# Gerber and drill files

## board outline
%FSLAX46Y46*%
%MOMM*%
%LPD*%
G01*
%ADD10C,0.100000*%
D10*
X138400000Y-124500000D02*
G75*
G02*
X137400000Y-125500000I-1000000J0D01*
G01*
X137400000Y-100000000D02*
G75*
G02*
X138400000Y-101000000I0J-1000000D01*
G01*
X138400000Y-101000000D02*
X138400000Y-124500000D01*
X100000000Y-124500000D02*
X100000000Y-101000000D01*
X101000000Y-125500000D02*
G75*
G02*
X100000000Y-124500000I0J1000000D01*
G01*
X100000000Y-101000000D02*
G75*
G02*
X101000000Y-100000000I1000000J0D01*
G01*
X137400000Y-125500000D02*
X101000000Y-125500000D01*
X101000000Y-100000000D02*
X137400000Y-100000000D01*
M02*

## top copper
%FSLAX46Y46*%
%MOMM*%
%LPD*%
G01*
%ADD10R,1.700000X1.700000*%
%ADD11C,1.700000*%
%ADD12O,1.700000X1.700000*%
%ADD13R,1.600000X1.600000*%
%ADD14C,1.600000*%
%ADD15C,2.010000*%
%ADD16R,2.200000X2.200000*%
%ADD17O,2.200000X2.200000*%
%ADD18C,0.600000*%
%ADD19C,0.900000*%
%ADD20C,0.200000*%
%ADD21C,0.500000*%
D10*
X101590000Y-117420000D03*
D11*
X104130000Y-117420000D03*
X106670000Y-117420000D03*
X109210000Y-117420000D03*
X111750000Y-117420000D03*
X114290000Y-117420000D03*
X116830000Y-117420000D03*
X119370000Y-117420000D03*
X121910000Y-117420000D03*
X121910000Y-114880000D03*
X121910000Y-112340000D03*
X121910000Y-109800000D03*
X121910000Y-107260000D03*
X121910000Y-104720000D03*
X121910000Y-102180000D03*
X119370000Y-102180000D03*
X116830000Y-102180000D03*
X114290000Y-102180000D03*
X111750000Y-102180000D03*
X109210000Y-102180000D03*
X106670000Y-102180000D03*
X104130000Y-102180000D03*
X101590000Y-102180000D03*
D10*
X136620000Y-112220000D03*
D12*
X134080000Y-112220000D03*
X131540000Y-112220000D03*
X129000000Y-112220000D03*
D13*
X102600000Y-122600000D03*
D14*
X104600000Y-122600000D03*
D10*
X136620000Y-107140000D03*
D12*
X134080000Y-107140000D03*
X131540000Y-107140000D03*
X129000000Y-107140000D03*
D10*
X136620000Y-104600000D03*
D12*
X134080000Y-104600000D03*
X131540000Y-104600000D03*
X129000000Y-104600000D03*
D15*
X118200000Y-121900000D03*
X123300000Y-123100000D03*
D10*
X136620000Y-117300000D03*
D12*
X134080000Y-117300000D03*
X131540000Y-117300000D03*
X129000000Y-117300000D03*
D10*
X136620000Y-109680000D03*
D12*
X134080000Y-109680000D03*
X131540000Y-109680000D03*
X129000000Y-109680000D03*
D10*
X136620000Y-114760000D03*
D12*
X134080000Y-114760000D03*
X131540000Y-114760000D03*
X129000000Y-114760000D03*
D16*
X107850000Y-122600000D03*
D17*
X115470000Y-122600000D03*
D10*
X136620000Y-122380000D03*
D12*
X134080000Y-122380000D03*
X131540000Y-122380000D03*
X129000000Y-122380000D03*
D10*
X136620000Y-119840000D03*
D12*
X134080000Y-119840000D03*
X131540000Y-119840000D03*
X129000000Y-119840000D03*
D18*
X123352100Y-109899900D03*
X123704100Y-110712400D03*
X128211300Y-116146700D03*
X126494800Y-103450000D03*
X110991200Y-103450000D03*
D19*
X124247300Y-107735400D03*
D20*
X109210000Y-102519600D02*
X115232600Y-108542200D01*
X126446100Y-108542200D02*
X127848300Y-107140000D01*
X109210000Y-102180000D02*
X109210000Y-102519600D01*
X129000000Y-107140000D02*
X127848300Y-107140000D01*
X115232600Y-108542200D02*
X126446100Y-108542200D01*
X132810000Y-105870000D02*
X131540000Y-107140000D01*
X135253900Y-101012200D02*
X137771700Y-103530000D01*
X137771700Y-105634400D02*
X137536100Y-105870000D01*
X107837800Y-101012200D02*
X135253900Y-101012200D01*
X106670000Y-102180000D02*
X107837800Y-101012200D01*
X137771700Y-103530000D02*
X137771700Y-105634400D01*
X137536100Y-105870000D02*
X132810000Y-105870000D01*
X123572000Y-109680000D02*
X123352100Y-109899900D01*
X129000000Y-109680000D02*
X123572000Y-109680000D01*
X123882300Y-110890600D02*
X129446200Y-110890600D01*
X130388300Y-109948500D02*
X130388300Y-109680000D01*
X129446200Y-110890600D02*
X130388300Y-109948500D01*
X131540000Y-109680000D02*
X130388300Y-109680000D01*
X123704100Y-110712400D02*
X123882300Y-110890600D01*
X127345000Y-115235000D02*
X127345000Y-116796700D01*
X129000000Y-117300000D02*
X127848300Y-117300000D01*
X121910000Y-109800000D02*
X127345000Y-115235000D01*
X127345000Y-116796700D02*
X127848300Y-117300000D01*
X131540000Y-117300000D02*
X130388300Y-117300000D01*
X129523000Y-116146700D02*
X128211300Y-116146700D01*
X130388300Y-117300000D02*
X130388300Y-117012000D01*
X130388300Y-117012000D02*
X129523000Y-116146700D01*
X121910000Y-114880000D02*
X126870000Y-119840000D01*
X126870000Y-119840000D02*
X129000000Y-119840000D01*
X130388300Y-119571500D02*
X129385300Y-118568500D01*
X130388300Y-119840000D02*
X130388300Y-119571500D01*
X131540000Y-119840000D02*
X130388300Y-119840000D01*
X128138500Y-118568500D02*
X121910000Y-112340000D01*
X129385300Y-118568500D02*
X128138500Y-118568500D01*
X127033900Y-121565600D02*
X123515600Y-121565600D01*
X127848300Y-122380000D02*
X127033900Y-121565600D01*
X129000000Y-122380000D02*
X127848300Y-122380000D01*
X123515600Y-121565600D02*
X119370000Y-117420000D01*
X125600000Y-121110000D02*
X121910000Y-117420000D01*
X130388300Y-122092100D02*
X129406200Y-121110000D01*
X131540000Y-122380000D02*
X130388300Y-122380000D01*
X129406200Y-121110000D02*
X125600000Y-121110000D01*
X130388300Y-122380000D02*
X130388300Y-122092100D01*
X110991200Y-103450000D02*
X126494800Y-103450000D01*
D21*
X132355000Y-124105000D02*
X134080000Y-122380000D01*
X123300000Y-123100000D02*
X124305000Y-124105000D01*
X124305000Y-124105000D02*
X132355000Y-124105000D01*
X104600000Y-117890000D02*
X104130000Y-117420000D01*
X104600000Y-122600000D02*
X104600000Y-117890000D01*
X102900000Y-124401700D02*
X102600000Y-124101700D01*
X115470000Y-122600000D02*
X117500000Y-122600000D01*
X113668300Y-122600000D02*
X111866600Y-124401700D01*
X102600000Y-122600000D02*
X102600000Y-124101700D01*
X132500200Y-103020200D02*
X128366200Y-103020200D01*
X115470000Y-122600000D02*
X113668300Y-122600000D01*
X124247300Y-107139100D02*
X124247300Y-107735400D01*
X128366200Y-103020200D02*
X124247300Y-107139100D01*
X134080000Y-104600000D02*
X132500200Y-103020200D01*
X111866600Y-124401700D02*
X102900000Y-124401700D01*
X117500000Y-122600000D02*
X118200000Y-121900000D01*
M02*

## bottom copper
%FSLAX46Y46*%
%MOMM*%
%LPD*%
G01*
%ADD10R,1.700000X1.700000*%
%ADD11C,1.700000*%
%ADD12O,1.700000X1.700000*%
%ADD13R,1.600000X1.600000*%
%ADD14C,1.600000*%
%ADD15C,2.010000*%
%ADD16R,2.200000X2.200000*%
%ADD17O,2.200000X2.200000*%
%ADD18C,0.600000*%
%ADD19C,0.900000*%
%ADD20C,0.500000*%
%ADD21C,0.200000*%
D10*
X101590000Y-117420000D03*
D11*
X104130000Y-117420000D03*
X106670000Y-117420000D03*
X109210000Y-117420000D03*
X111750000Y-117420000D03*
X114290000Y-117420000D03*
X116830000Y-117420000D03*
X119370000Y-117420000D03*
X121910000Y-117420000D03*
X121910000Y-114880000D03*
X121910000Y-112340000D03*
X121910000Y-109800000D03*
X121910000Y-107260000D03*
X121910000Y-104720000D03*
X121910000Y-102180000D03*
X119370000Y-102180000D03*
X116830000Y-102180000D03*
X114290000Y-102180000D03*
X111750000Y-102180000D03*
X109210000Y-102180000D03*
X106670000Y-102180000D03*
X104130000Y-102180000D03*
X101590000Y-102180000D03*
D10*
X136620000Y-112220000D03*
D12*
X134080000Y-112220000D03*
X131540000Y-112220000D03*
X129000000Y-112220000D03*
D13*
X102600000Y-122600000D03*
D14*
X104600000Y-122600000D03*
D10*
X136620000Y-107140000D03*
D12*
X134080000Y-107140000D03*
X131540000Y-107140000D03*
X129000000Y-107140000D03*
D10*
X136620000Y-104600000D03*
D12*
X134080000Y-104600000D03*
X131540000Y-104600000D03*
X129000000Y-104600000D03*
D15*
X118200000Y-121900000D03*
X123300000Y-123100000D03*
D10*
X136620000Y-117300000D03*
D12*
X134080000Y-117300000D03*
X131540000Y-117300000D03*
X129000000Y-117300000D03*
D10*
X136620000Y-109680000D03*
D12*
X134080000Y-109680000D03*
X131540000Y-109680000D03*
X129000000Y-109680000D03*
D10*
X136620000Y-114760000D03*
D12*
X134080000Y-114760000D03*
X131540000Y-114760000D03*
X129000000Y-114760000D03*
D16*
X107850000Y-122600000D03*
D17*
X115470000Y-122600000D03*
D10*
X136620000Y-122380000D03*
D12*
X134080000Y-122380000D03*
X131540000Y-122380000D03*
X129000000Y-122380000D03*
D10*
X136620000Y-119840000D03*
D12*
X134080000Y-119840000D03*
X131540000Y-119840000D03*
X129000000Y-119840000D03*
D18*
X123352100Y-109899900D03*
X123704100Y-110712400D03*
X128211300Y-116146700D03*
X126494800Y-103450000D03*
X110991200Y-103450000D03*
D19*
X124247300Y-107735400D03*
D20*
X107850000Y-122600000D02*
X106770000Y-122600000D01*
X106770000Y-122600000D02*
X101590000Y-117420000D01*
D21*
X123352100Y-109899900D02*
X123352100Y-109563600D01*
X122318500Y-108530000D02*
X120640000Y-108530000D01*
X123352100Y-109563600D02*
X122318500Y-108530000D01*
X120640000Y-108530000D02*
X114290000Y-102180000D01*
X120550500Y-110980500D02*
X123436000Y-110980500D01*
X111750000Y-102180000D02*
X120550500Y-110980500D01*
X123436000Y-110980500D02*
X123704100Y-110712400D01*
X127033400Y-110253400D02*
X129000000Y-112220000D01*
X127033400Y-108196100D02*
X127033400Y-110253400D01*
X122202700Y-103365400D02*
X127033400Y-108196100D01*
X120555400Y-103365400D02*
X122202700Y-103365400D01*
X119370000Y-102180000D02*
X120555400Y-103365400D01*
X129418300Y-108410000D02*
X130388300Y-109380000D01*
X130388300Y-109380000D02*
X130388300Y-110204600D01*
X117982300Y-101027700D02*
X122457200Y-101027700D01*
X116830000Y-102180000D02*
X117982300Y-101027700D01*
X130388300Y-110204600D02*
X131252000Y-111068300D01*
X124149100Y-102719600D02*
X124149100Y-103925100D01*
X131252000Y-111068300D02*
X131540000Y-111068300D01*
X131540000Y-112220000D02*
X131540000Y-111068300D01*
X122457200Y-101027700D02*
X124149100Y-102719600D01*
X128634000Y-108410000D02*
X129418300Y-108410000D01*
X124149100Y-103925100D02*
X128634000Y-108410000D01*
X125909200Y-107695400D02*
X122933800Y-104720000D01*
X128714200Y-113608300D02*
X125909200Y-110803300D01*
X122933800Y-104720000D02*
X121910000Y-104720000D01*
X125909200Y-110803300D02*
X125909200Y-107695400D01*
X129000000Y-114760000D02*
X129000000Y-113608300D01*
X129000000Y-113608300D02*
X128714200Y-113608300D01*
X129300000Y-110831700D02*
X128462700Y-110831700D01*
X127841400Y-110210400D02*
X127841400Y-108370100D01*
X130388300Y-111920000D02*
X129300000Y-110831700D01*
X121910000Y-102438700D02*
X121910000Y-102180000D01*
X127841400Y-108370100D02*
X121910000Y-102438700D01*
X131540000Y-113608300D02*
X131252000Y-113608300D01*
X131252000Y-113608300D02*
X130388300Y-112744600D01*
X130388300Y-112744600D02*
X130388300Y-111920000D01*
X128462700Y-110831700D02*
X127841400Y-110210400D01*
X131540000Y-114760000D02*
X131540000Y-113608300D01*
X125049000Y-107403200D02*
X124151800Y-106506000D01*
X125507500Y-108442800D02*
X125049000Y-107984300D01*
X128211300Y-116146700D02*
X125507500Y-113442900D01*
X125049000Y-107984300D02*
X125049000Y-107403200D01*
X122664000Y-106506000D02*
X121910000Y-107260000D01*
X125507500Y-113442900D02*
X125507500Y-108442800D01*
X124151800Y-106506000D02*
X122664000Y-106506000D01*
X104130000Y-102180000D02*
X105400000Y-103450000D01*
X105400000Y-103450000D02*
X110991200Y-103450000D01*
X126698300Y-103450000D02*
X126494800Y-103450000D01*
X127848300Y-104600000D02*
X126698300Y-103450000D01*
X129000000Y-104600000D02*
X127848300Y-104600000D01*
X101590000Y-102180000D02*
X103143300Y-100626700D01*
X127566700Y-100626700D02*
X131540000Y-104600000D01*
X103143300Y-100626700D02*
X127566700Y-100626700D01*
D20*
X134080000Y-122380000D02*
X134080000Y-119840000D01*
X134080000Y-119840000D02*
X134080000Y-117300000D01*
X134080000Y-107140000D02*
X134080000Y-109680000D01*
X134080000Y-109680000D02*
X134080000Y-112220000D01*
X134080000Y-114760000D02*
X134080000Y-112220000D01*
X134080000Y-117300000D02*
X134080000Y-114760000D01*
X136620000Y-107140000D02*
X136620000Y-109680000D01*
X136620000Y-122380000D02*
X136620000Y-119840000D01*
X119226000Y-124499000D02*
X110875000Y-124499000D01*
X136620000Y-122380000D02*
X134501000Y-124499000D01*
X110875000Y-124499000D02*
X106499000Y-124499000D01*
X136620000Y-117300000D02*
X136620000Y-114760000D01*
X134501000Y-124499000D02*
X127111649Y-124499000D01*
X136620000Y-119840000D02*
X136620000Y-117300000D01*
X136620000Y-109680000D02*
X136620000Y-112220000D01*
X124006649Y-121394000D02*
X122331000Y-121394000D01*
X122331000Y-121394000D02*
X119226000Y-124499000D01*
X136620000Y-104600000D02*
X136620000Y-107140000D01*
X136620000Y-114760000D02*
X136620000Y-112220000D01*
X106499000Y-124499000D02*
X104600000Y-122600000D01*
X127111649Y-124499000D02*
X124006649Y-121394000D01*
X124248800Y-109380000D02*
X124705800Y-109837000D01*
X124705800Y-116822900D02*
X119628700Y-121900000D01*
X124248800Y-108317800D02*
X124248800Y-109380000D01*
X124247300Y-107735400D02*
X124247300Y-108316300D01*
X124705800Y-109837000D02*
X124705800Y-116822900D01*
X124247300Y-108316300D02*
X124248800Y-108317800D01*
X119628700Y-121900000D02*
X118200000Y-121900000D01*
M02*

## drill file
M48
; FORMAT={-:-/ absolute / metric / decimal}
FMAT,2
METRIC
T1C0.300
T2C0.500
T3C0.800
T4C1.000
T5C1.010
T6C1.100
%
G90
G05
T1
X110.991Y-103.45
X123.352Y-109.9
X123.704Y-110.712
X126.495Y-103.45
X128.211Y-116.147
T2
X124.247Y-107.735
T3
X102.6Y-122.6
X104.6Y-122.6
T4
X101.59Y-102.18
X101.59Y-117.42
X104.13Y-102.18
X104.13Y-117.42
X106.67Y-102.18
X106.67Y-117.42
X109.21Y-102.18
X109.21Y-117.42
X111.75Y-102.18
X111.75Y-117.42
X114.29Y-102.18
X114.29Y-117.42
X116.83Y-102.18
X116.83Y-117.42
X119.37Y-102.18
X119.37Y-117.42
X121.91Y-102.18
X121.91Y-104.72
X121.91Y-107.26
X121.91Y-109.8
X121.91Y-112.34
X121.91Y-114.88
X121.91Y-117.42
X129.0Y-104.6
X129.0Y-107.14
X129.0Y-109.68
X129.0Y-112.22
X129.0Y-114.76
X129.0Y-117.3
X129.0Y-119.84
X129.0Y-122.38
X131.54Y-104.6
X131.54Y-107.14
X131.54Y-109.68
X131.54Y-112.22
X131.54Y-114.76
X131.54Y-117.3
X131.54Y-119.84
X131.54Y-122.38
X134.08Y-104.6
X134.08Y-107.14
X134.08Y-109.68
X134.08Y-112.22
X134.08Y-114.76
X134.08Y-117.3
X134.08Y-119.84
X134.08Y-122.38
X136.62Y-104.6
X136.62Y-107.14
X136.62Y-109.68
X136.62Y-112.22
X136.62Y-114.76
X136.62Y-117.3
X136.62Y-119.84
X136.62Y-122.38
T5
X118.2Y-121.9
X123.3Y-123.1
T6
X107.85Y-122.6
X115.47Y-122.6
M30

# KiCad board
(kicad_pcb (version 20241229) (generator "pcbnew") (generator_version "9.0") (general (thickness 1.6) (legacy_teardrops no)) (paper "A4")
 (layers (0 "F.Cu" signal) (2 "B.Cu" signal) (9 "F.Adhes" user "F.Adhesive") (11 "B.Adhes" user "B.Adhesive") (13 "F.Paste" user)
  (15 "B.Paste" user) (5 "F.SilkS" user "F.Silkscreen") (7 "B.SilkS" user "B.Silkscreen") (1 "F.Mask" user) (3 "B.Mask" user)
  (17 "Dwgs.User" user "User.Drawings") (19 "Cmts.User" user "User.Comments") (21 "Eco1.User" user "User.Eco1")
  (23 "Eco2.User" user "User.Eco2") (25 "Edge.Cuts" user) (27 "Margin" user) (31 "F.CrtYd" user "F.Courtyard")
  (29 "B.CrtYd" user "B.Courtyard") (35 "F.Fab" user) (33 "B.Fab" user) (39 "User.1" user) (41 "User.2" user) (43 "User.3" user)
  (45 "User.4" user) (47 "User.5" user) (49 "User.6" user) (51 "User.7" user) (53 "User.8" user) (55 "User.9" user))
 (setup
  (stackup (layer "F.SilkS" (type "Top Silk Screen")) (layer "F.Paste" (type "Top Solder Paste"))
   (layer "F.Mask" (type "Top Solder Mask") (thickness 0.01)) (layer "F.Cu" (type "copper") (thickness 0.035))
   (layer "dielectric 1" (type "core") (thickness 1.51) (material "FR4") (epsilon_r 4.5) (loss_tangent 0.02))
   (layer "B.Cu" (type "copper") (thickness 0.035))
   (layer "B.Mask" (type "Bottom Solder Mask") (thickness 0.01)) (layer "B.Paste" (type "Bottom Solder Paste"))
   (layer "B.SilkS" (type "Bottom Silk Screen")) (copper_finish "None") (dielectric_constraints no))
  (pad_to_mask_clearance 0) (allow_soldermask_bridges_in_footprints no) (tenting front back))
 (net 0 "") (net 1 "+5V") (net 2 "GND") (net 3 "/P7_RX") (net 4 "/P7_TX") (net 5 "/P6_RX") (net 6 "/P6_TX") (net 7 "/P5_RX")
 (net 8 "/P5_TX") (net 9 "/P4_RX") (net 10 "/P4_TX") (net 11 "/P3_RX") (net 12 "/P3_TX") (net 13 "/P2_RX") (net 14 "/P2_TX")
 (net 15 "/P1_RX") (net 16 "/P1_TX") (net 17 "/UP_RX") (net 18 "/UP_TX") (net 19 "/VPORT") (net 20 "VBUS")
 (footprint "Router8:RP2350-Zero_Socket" (layer "F.Cu") (at 111.75 109.8 90)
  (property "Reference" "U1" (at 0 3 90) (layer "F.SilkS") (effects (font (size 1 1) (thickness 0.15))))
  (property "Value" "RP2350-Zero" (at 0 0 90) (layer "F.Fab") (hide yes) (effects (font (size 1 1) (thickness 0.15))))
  (pad "1" thru_hole rect (at -7.62 -10.16 90) (size 1.7 1.7) (drill 1) (layers "*.Cu" "*.Mask") (remove_unused_layers no) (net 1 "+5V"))
  (pad "2" thru_hole circle (at -7.62 -7.62 90) (size 1.7 1.7) (drill 1) (layers "*.Cu" "*.Mask") (remove_unused_layers no) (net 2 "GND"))
  (pad "3" thru_hole circle (at -7.62 -5.08 90) (size 1.7 1.7) (drill 1) (layers "*.Cu" "*.Mask") (remove_unused_layers no))
  (pad "4" thru_hole circle (at -7.62 -2.54 90) (size 1.7 1.7) (drill 1) (layers "*.Cu" "*.Mask") (remove_unused_layers no))
  (pad "5" thru_hole circle (at -7.62 0 90) (size 1.7 1.7) (drill 1) (layers "*.Cu" "*.Mask") (remove_unused_layers no))
  (pad "6" thru_hole circle (at -7.62 2.54 90) (size 1.7 1.7) (drill 1) (layers "*.Cu" "*.Mask") (remove_unused_layers no))
  (pad "7" thru_hole circle (at -7.62 5.08 90) (size 1.7 1.7) (drill 1) (layers "*.Cu" "*.Mask") (remove_unused_layers no))
  (pad "8" thru_hole circle (at -7.62 7.62 90) (size 1.7 1.7) (drill 1) (layers "*.Cu" "*.Mask") (remove_unused_layers no) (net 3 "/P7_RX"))
  (pad "9" thru_hole circle (at -7.62 10.16 90) (size 1.7 1.7) (drill 1) (layers "*.Cu" "*.Mask") (remove_unused_layers no) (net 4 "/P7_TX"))
  (pad "10" thru_hole circle (at -5.08 10.16 90) (size 1.7 1.7) (drill 1) (layers "*.Cu" "*.Mask") (remove_unused_layers no)
   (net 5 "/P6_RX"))
  (pad "11" thru_hole circle (at -2.54 10.16 90) (size 1.7 1.7) (drill 1) (layers "*.Cu" "*.Mask") (remove_unused_layers no)
   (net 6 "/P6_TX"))
  (pad "12" thru_hole circle (at 0 10.16 90) (size 1.7 1.7) (drill 1) (layers "*.Cu" "*.Mask") (remove_unused_layers no) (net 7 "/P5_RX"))
  (pad "13" thru_hole circle (at 2.54 10.16 90) (size 1.7 1.7) (drill 1) (layers "*.Cu" "*.Mask") (remove_unused_layers no) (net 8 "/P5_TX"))
  (pad "14" thru_hole circle (at 5.08 10.16 90) (size 1.7 1.7) (drill 1) (layers "*.Cu" "*.Mask") (remove_unused_layers no) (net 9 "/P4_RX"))
  (pad "15" thru_hole circle (at 7.62 10.16 90) (size 1.7 1.7) (drill 1) (layers "*.Cu" "*.Mask") (remove_unused_layers no)
   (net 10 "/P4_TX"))
  (pad "16" thru_hole circle (at 7.62 7.62 90) (size 1.7 1.7) (drill 1) (layers "*.Cu" "*.Mask") (remove_unused_layers no) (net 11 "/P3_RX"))
  (pad "17" thru_hole circle (at 7.62 5.08 90) (size 1.7 1.7) (drill 1) (layers "*.Cu" "*.Mask") (remove_unused_layers no) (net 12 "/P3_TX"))
  (pad "18" thru_hole circle (at 7.62 2.54 90) (size 1.7 1.7) (drill 1) (layers "*.Cu" "*.Mask") (remove_unused_layers no) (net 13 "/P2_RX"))
  (pad "19" thru_hole circle (at 7.62 0 90) (size 1.7 1.7) (drill 1) (layers "*.Cu" "*.Mask") (remove_unused_layers no) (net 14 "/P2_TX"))
  (pad "20" thru_hole circle (at 7.62 -2.54 90) (size 1.7 1.7) (drill 1) (layers "*.Cu" "*.Mask") (remove_unused_layers no)
   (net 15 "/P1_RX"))
  (pad "21" thru_hole circle (at 7.62 -5.08 90) (size 1.7 1.7) (drill 1) (layers "*.Cu" "*.Mask") (remove_unused_layers no)
   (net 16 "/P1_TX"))
  (pad "22" thru_hole circle (at 7.62 -7.62 90) (size 1.7 1.7) (drill 1) (layers "*.Cu" "*.Mask") (remove_unused_layers no)
   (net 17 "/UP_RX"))
  (pad "23" thru_hole circle (at 7.62 -10.16 90) (size 1.7 1.7) (drill 1) (layers "*.Cu" "*.Mask") (remove_unused_layers no)
   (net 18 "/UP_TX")))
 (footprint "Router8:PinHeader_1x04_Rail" (layer "F.Cu") (at 136.62 112.22 -90)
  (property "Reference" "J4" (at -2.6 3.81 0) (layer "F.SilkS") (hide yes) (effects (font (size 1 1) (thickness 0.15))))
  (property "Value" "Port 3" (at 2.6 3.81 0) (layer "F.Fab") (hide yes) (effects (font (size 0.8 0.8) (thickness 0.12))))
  (pad "1" thru_hole rect (at 0 0 270) (size 1.7 1.7) (drill 1) (layers "*.Cu" "*.Mask") (remove_unused_layers no) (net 2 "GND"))
  (pad "2" thru_hole oval (at 0 2.54 270) (size 1.7 1.7) (drill 1) (layers "*.Cu" "*.Mask") (remove_unused_layers no) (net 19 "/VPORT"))
  (pad "3" thru_hole oval (at 0 5.08 270) (size 1.7 1.7) (drill 1) (layers "*.Cu" "*.Mask") (remove_unused_layers no) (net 12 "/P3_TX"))
  (pad "4" thru_hole oval (at 0 7.62 270) (size 1.7 1.7) (drill 1) (layers "*.Cu" "*.Mask") (remove_unused_layers no) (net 11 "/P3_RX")))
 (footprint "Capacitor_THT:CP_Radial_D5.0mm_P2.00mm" (layer "F.Cu") (at 102.6 122.6)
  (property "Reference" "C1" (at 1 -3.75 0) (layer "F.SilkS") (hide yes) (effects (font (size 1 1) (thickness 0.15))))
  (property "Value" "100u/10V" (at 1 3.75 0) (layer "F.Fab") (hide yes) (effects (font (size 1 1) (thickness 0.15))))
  (pad "1" thru_hole rect (at 0 0) (size 1.6 1.6) (drill 0.8) (layers "*.Cu" "*.Mask") (remove_unused_layers no) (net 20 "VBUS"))
  (pad "2" thru_hole circle (at 2 0) (size 1.6 1.6) (drill 0.8) (layers "*.Cu" "*.Mask") (remove_unused_layers no) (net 2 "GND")))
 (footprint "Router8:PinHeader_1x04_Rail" (layer "F.Cu") (at 136.62 107.14 -90)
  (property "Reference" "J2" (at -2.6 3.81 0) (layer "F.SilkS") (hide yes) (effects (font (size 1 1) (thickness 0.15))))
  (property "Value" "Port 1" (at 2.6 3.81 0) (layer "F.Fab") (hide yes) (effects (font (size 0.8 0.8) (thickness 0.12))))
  (pad "1" thru_hole rect (at 0 0 270) (size 1.7 1.7) (drill 1) (layers "*.Cu" "*.Mask") (remove_unused_layers no) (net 2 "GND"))
  (pad "2" thru_hole oval (at 0 2.54 270) (size 1.7 1.7) (drill 1) (layers "*.Cu" "*.Mask") (remove_unused_layers no) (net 19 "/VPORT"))
  (pad "3" thru_hole oval (at 0 5.08 270) (size 1.7 1.7) (drill 1) (layers "*.Cu" "*.Mask") (remove_unused_layers no) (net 16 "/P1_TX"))
  (pad "4" thru_hole oval (at 0 7.62 270) (size 1.7 1.7) (drill 1) (layers "*.Cu" "*.Mask") (remove_unused_layers no) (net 15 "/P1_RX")))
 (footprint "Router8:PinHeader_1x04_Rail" (layer "F.Cu") (at 136.62 104.6 -90)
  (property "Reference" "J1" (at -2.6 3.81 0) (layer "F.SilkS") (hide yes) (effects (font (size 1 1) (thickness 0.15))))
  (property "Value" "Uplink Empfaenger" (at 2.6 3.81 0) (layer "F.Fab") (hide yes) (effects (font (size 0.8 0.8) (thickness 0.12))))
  (pad "1" thru_hole rect (at 0 0 270) (size 1.7 1.7) (drill 1) (layers "*.Cu" "*.Mask") (remove_unused_layers no) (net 2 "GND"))
  (pad "2" thru_hole oval (at 0 2.54 270) (size 1.7 1.7) (drill 1) (layers "*.Cu" "*.Mask") (remove_unused_layers no) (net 20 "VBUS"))
  (pad "3" thru_hole oval (at 0 5.08 270) (size 1.7 1.7) (drill 1) (layers "*.Cu" "*.Mask") (remove_unused_layers no) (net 18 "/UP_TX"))
  (pad "4" thru_hole oval (at 0 7.62 270) (size 1.7 1.7) (drill 1) (layers "*.Cu" "*.Mask") (remove_unused_layers no) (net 17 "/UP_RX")))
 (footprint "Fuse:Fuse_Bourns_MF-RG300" (layer "F.Cu") (at 118.2 121.9)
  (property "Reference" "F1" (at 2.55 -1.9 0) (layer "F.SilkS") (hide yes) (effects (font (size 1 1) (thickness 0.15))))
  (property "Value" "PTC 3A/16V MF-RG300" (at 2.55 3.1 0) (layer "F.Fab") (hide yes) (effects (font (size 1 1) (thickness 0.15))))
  (pad "1" thru_hole circle (at 0 0) (size 2.01 2.01) (drill 1.01) (layers "*.Cu" "*.Mask") (remove_unused_layers no) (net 20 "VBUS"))
  (pad "2" thru_hole circle (at 5.1 1.2) (size 2.01 2.01) (drill 1.01) (layers "*.Cu" "*.Mask") (remove_unused_layers no) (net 19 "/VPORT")))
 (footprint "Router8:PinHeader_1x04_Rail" (layer "F.Cu") (at 136.62 117.3 -90)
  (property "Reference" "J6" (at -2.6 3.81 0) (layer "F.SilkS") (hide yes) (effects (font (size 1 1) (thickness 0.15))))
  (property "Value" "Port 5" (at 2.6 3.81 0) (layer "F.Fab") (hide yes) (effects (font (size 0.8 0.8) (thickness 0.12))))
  (pad "1" thru_hole rect (at 0 0 270) (size 1.7 1.7) (drill 1) (layers "*.Cu" "*.Mask") (remove_unused_layers no) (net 2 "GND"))
  (pad "2" thru_hole oval (at 0 2.54 270) (size 1.7 1.7) (drill 1) (layers "*.Cu" "*.Mask") (remove_unused_layers no) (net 19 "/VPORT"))
  (pad "3" thru_hole oval (at 0 5.08 270) (size 1.7 1.7) (drill 1) (layers "*.Cu" "*.Mask") (remove_unused_layers no) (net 8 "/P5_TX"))
  (pad "4" thru_hole oval (at 0 7.62 270) (size 1.7 1.7) (drill 1) (layers "*.Cu" "*.Mask") (remove_unused_layers no) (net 7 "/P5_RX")))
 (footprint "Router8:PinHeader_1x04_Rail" (layer "F.Cu") (at 136.62 109.68 -90)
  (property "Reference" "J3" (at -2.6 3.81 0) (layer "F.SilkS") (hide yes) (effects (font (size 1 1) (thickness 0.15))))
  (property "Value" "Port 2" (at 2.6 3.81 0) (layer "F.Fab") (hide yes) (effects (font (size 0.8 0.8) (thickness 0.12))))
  (pad "1" thru_hole rect (at 0 0 270) (size 1.7 1.7) (drill 1) (layers "*.Cu" "*.Mask") (remove_unused_layers no) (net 2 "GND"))
  (pad "2" thru_hole oval (at 0 2.54 270) (size 1.7 1.7) (drill 1) (layers "*.Cu" "*.Mask") (remove_unused_layers no) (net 19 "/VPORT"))
  (pad "3" thru_hole oval (at 0 5.08 270) (size 1.7 1.7) (drill 1) (layers "*.Cu" "*.Mask") (remove_unused_layers no) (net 14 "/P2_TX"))
  (pad "4" thru_hole oval (at 0 7.62 270) (size 1.7 1.7) (drill 1) (layers "*.Cu" "*.Mask") (remove_unused_layers no) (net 13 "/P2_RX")))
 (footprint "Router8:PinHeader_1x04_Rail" (layer "F.Cu") (at 136.62 114.76 -90)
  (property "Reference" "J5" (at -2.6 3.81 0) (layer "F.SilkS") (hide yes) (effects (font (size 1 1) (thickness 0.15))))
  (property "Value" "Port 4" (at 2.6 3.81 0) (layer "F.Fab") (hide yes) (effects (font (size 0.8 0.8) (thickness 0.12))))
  (pad "1" thru_hole rect (at 0 0 270) (size 1.7 1.7) (drill 1) (layers "*.Cu" "*.Mask") (remove_unused_layers no) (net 2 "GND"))
  (pad "2" thru_hole oval (at 0 2.54 270) (size 1.7 1.7) (drill 1) (layers "*.Cu" "*.Mask") (remove_unused_layers no) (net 19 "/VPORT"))
  (pad "3" thru_hole oval (at 0 5.08 270) (size 1.7 1.7) (drill 1) (layers "*.Cu" "*.Mask") (remove_unused_layers no) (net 10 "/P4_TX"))
  (pad "4" thru_hole oval (at 0 7.62 270) (size 1.7 1.7) (drill 1) (layers "*.Cu" "*.Mask") (remove_unused_layers no) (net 9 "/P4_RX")))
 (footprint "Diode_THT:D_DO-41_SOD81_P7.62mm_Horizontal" (layer "F.Cu") (at 107.85 122.6)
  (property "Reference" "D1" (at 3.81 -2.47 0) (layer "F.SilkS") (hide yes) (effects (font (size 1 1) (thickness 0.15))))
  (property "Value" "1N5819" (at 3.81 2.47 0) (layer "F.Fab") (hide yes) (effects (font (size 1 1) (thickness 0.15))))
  (pad "1" thru_hole rect (at 0 0) (size 2.2 2.2) (drill 1.1) (layers "*.Cu" "*.Mask") (remove_unused_layers no) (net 1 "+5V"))
  (pad "2" thru_hole oval (at 7.62 0) (size 2.2 2.2) (drill 1.1) (layers "*.Cu" "*.Mask") (remove_unused_layers no) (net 20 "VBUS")))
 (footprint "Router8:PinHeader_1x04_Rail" (layer "F.Cu") (at 136.62 122.38 -90)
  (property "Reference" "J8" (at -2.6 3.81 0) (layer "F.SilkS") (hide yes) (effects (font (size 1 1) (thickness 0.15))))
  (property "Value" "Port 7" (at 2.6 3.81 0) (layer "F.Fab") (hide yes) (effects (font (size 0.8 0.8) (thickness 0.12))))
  (pad "1" thru_hole rect (at 0 0 270) (size 1.7 1.7) (drill 1) (layers "*.Cu" "*.Mask") (remove_unused_layers no) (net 2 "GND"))
  (pad "2" thru_hole oval (at 0 2.54 270) (size 1.7 1.7) (drill 1) (layers "*.Cu" "*.Mask") (remove_unused_layers no) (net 19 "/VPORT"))
  (pad "3" thru_hole oval (at 0 5.08 270) (size 1.7 1.7) (drill 1) (layers "*.Cu" "*.Mask") (remove_unused_layers no) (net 4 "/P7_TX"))
  (pad "4" thru_hole oval (at 0 7.62 270) (size 1.7 1.7) (drill 1) (layers "*.Cu" "*.Mask") (remove_unused_layers no) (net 3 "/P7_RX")))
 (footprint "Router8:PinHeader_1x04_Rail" (layer "F.Cu") (at 136.62 119.84 -90)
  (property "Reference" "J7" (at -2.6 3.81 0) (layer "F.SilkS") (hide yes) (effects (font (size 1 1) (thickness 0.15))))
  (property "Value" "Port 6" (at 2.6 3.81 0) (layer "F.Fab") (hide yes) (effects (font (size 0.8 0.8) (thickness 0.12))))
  (pad "1" thru_hole rect (at 0 0 270) (size 1.7 1.7) (drill 1) (layers "*.Cu" "*.Mask") (remove_unused_layers no) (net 2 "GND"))
  (pad "2" thru_hole oval (at 0 2.54 270) (size 1.7 1.7) (drill 1) (layers "*.Cu" "*.Mask") (remove_unused_layers no) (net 19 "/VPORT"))
  (pad "3" thru_hole oval (at 0 5.08 270) (size 1.7 1.7) (drill 1) (layers "*.Cu" "*.Mask") (remove_unused_layers no) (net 6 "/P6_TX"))
  (pad "4" thru_hole oval (at 0 7.62 270) (size 1.7 1.7) (drill 1) (layers "*.Cu" "*.Mask") (remove_unused_layers no) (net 5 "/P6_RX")))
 (gr_arc (start 138.4 124.5) (mid 138.107107 125.207107) (end 137.4 125.5) (stroke (width 0.1) (type default)) (layer "Edge.Cuts"))
 (gr_arc (start 137.4 100) (mid 138.107107 100.292893) (end 138.4 101) (stroke (width 0.1) (type default)) (layer "Edge.Cuts"))
 (gr_line (start 138.4 101) (end 138.4 124.5) (stroke (width 0.1) (type default)) (layer "Edge.Cuts"))
 (gr_line (start 100 124.5) (end 100 101) (stroke (width 0.1) (type default)) (layer "Edge.Cuts"))
 (gr_arc (start 101 125.5) (mid 100.292893 125.207107) (end 100 124.5) (stroke (width 0.1) (type default)) (layer "Edge.Cuts"))
 (gr_arc (start 100 101) (mid 100.292893 100.292893) (end 101 100) (stroke (width 0.1) (type default)) (layer "Edge.Cuts"))
 (gr_line (start 137.4 125.5) (end 101 125.5) (stroke (width 0.1) (type default)) (layer "Edge.Cuts"))
 (gr_line (start 101 100) (end 137.4 100) (stroke (width 0.1) (type default)) (layer "Edge.Cuts"))
 (segment (start 107.85 122.6) (end 106.77 122.6) (width 0.5) (layer "B.Cu") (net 1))
 (segment (start 106.77 122.6) (end 101.59 117.42) (width 0.5) (layer "B.Cu") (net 1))
 (segment (start 109.21 102.5196) (end 115.2326 108.5422) (width 0.2) (layer "F.Cu") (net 15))
 (segment (start 126.4461 108.5422) (end 127.8483 107.14) (width 0.2) (layer "F.Cu") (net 15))
 (segment (start 109.21 102.18) (end 109.21 102.5196) (width 0.2) (layer "F.Cu") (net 15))
 (segment (start 129 107.14) (end 127.8483 107.14) (width 0.2) (layer "F.Cu") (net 15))
 (segment (start 115.2326 108.5422) (end 126.4461 108.5422) (width 0.2) (layer "F.Cu") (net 15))
 (segment (start 132.81 105.87) (end 131.54 107.14) (width 0.2) (layer "F.Cu") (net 16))
 (segment (start 135.2539 101.0122) (end 137.7717 103.53) (width 0.2) (layer "F.Cu") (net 16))
 (segment (start 137.7717 105.6344) (end 137.5361 105.87) (width 0.2) (layer "F.Cu") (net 16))
 (segment (start 107.8378 101.0122) (end 135.2539 101.0122) (width 0.2) (layer "F.Cu") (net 16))
 (segment (start 106.67 102.18) (end 107.8378 101.0122) (width 0.2) (layer "F.Cu") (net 16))
 (segment (start 137.7717 103.53) (end 137.7717 105.6344) (width 0.2) (layer "F.Cu") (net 16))
 (segment (start 137.5361 105.87) (end 132.81 105.87) (width 0.2) (layer "F.Cu") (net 16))
 (segment (start 123.572 109.68) (end 123.3521 109.8999) (width 0.2) (layer "F.Cu") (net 13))
 (segment (start 129 109.68) (end 123.572 109.68) (width 0.2) (layer "F.Cu") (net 13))
 (via (at 123.3521 109.8999) (size 0.6) (drill 0.3) (layers "F.Cu" "B.Cu") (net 13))
 (segment (start 123.3521 109.8999) (end 123.3521 109.5636) (width 0.2) (layer "B.Cu") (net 13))
 (segment (start 122.3185 108.53) (end 120.64 108.53) (width 0.2) (layer "B.Cu") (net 13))
 (segment (start 123.3521 109.5636) (end 122.3185 108.53) (width 0.2) (layer "B.Cu") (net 13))
 (segment (start 120.64 108.53) (end 114.29 102.18) (width 0.2) (layer "B.Cu") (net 13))
 (segment (start 123.8823 110.8906) (end 129.4462 110.8906) (width 0.2) (layer "F.Cu") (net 14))
 (segment (start 130.3883 109.9485) (end 130.3883 109.68) (width 0.2) (layer "F.Cu") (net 14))
 (segment (start 129.4462 110.8906) (end 130.3883 109.9485) (width 0.2) (layer "F.Cu") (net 14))
 (segment (start 131.54 109.68) (end 130.3883 109.68) (width 0.2) (layer "F.Cu") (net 14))
 (segment (start 123.7041 110.7124) (end 123.8823 110.8906) (width 0.2) (layer "F.Cu") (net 14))
 (via (at 123.7041 110.7124) (size 0.6) (drill 0.3) (layers "F.Cu" "B.Cu") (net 14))
 (segment (start 120.5505 110.9805) (end 123.436 110.9805) (width 0.2) (layer "B.Cu") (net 14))
 (segment (start 111.75 102.18) (end 120.5505 110.9805) (width 0.2) (layer "B.Cu") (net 14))
 (segment (start 123.436 110.9805) (end 123.7041 110.7124) (width 0.2) (layer "B.Cu") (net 14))
 (segment (start 127.0334 110.2534) (end 129 112.22) (width 0.2) (layer "B.Cu") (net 11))
 (segment (start 127.0334 108.1961) (end 127.0334 110.2534) (width 0.2) (layer "B.Cu") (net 11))
 (segment (start 122.2027 103.3654) (end 127.0334 108.1961) (width 0.2) (layer "B.Cu") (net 11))
 (segment (start 120.5554 103.3654) (end 122.2027 103.3654) (width 0.2) (layer "B.Cu") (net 11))
 (segment (start 119.37 102.18) (end 120.5554 103.3654) (width 0.2) (layer "B.Cu") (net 11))
 (segment (start 129.4183 108.41) (end 130.3883 109.38) (width 0.2) (layer "B.Cu") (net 12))
 (segment (start 130.3883 109.38) (end 130.3883 110.2046) (width 0.2) (layer "B.Cu") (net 12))
 (segment (start 117.9823 101.0277) (end 122.4572 101.0277) (width 0.2) (layer "B.Cu") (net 12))
 (segment (start 116.83 102.18) (end 117.9823 101.0277) (width 0.2) (layer "B.Cu") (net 12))
 (segment (start 130.3883 110.2046) (end 131.252 111.0683) (width 0.2) (layer "B.Cu") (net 12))
 (segment (start 124.1491 102.7196) (end 124.1491 103.9251) (width 0.2) (layer "B.Cu") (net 12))
 (segment (start 131.252 111.0683) (end 131.54 111.0683) (width 0.2) (layer "B.Cu") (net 12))
 (segment (start 131.54 112.22) (end 131.54 111.0683) (width 0.2) (layer "B.Cu") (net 12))
 (segment (start 122.4572 101.0277) (end 124.1491 102.7196) (width 0.2) (layer "B.Cu") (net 12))
 (segment (start 128.634 108.41) (end 129.4183 108.41) (width 0.2) (layer "B.Cu") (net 12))
 (segment (start 124.1491 103.9251) (end 128.634 108.41) (width 0.2) (layer "B.Cu") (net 12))
 (segment (start 125.9092 107.6954) (end 122.9338 104.72) (width 0.2) (layer "B.Cu") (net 9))
 (segment (start 128.7142 113.6083) (end 125.9092 110.8033) (width 0.2) (layer "B.Cu") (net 9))
 (segment (start 122.9338 104.72) (end 121.91 104.72) (width 0.2) (layer "B.Cu") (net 9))
 (segment (start 125.9092 110.8033) (end 125.9092 107.6954) (width 0.2) (layer "B.Cu") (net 9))
 (segment (start 129 114.76) (end 129 113.6083) (width 0.2) (layer "B.Cu") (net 9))
 (segment (start 129 113.6083) (end 128.7142 113.6083) (width 0.2) (layer "B.Cu") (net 9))
 (segment (start 129.3 110.8317) (end 128.4627 110.8317) (width 0.2) (layer "B.Cu") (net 10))
 (segment (start 127.8414 110.2104) (end 127.8414 108.3701) (width 0.2) (layer "B.Cu") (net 10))
 (segment (start 130.3883 111.92) (end 129.3 110.8317) (width 0.2) (layer "B.Cu") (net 10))
 (segment (start 121.91 102.4387) (end 121.91 102.18) (width 0.2) (layer "B.Cu") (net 10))
 (segment (start 127.8414 108.3701) (end 121.91 102.4387) (width 0.2) (layer "B.Cu") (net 10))
 (segment (start 131.54 113.6083) (end 131.252 113.6083) (width 0.2) (layer "B.Cu") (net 10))
 (segment (start 131.252 113.6083) (end 130.3883 112.7446) (width 0.2) (layer "B.Cu") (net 10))
 (segment (start 130.3883 112.7446) (end 130.3883 111.92) (width 0.2) (layer "B.Cu") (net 10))
 (segment (start 128.4627 110.8317) (end 127.8414 110.2104) (width 0.2) (layer "B.Cu") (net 10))
 (segment (start 131.54 114.76) (end 131.54 113.6083) (width 0.2) (layer "B.Cu") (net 10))
 (segment (start 127.345 115.235) (end 127.345 116.7967) (width 0.2) (layer "F.Cu") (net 7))
 (segment (start 129 117.3) (end 127.8483 117.3) (width 0.2) (layer "F.Cu") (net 7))
 (segment (start 121.91 109.8) (end 127.345 115.235) (width 0.2) (layer "F.Cu") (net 7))
 (segment (start 127.345 116.7967) (end 127.8483 117.3) (width 0.2) (layer "F.Cu") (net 7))
 (segment (start 131.54 117.3) (end 130.3883 117.3) (width 0.2) (layer "F.Cu") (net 8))
 (segment (start 129.523 116.1467) (end 128.2113 116.1467) (width 0.2) (layer "F.Cu") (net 8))
 (segment (start 130.3883 117.3) (end 130.3883 117.012) (width 0.2) (layer "F.Cu") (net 8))
 (segment (start 130.3883 117.012) (end 129.523 116.1467) (width 0.2) (layer "F.Cu") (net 8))
 (via (at 128.2113 116.1467) (size 0.6) (drill 0.3) (layers "F.Cu" "B.Cu") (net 8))
 (segment (start 125.049 107.4032) (end 124.1518 106.506) (width 0.2) (layer "B.Cu") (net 8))
 (segment (start 125.5075 108.4428) (end 125.049 107.9843) (width 0.2) (layer "B.Cu") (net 8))
 (segment (start 128.2113 116.1467) (end 125.5075 113.4429) (width 0.2) (layer "B.Cu") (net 8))
 (segment (start 125.049 107.9843) (end 125.049 107.4032) (width 0.2) (layer "B.Cu") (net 8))
 (segment (start 122.664 106.506) (end 121.91 107.26) (width 0.2) (layer "B.Cu") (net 8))
 (segment (start 125.5075 113.4429) (end 125.5075 108.4428) (width 0.2) (layer "B.Cu") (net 8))
 (segment (start 124.1518 106.506) (end 122.664 106.506) (width 0.2) (layer "B.Cu") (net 8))
 (segment (start 121.91 114.88) (end 126.87 119.84) (width 0.2) (layer "F.Cu") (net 5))
 (segment (start 126.87 119.84) (end 129 119.84) (width 0.2) (layer "F.Cu") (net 5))
 (segment (start 130.3883 119.5715) (end 129.3853 118.5685) (width 0.2) (layer "F.Cu") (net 6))
 (segment (start 130.3883 119.84) (end 130.3883 119.5715) (width 0.2) (layer "F.Cu") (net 6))
 (segment (start 131.54 119.84) (end 130.3883 119.84) (width 0.2) (layer "F.Cu") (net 6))
 (segment (start 128.1385 118.5685) (end 121.91 112.34) (width 0.2) (layer "F.Cu") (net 6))
 (segment (start 129.3853 118.5685) (end 128.1385 118.5685) (width 0.2) (layer "F.Cu") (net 6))
 (segment (start 127.0339 121.5656) (end 123.5156 121.5656) (width 0.2) (layer "F.Cu") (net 3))
 (segment (start 127.8483 122.38) (end 127.0339 121.5656) (width 0.2) (layer "F.Cu") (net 3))
 (segment (start 129 122.38) (end 127.8483 122.38) (width 0.2) (layer "F.Cu") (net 3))
 (segment (start 123.5156 121.5656) (end 119.37 117.42) (width 0.2) (layer "F.Cu") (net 3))
 (segment (start 125.6 121.11) (end 121.91 117.42) (width 0.2) (layer "F.Cu") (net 4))
 (segment (start 130.3883 122.0921) (end 129.4062 121.11) (width 0.2) (layer "F.Cu") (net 4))
 (segment (start 131.54 122.38) (end 130.3883 122.38) (width 0.2) (layer "F.Cu") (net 4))
 (segment (start 129.4062 121.11) (end 125.6 121.11) (width 0.2) (layer "F.Cu") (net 4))
 (segment (start 130.3883 122.38) (end 130.3883 122.0921) (width 0.2) (layer "F.Cu") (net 4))
 (segment (start 110.9912 103.45) (end 126.4948 103.45) (width 0.2) (layer "F.Cu") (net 17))
 (via (at 126.4948 103.45) (size 0.6) (drill 0.3) (layers "F.Cu" "B.Cu") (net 17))
 (via (at 110.9912 103.45) (size 0.6) (drill 0.3) (layers "F.Cu" "B.Cu") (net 17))
 (segment (start 104.13 102.18) (end 105.4 103.45) (width 0.2) (layer "B.Cu") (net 17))
 (segment (start 105.4 103.45) (end 110.9912 103.45) (width 0.2) (layer "B.Cu") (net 17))
 (segment (start 126.6983 103.45) (end 126.4948 103.45) (width 0.2) (layer "B.Cu") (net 17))
 (segment (start 127.8483 104.6) (end 126.6983 103.45) (width 0.2) (layer "B.Cu") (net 17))
 (segment (start 129 104.6) (end 127.8483 104.6) (width 0.2) (layer "B.Cu") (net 17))
 (segment (start 101.59 102.18) (end 103.1433 100.6267) (width 0.2) (layer "B.Cu") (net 18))
 (segment (start 127.5667 100.6267) (end 131.54 104.6) (width 0.2) (layer "B.Cu") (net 18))
 (segment (start 103.1433 100.6267) (end 127.5667 100.6267) (width 0.2) (layer "B.Cu") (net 18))
 (segment (start 132.355 124.105) (end 134.08 122.38) (width 0.5) (layer "F.Cu") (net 19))
 (segment (start 123.3 123.1) (end 124.305 124.105) (width 0.5) (layer "F.Cu") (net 19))
 (segment (start 124.305 124.105) (end 132.355 124.105) (width 0.5) (layer "F.Cu") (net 19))
 (segment (start 134.08 122.38) (end 134.08 119.84) (width 0.5) (layer "B.Cu") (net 19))
 (segment (start 134.08 119.84) (end 134.08 117.3) (width 0.5) (layer "B.Cu") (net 19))
 (segment (start 134.08 107.14) (end 134.08 109.68) (width 0.5) (layer "B.Cu") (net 19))
 (segment (start 134.08 109.68) (end 134.08 112.22) (width 0.5) (layer "B.Cu") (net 19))
 (segment (start 134.08 114.76) (end 134.08 112.22) (width 0.5) (layer "B.Cu") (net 19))
 (segment (start 134.08 117.3) (end 134.08 114.76) (width 0.5) (layer "B.Cu") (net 19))
 (segment (start 104.6 117.89) (end 104.13 117.42) (width 0.5) (layer "F.Cu") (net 2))
 (segment (start 104.6 122.6) (end 104.6 117.89) (width 0.5) (layer "F.Cu") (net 2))
 (segment (start 136.62 107.14) (end 136.62 109.68) (width 0.5) (layer "B.Cu") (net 2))
 (segment (start 136.62 122.38) (end 136.62 119.84) (width 0.5) (layer "B.Cu") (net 2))
 (segment (start 119.226 124.499) (end 110.875 124.499) (width 0.5) (layer "B.Cu") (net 2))
 (segment (start 136.62 122.38) (end 134.501 124.499) (width 0.5) (layer "B.Cu") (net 2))
 (segment (start 110.875 124.499) (end 106.499 124.499) (width 0.5) (layer "B.Cu") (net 2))
 (segment (start 136.62 117.3) (end 136.62 114.76) (width 0.5) (layer "B.Cu") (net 2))
 (segment (start 134.501 124.499) (end 127.111649 124.499) (width 0.5) (layer "B.Cu") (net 2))
 (segment (start 136.62 119.84) (end 136.62 117.3) (width 0.5) (layer "B.Cu") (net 2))
 (segment (start 136.62 109.68) (end 136.62 112.22) (width 0.5) (layer "B.Cu") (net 2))
 (segment (start 124.006649 121.394) (end 122.331 121.394) (width 0.5) (layer "B.Cu") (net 2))
 (segment (start 122.331 121.394) (end 119.226 124.499) (width 0.5) (layer "B.Cu") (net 2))
 (segment (start 136.62 104.6) (end 136.62 107.14) (width 0.5) (layer "B.Cu") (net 2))
 (segment (start 136.62 114.76) (end 136.62 112.22) (width 0.5) (layer "B.Cu") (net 2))
 (segment (start 106.499 124.499) (end 104.6 122.6) (width 0.5) (layer "B.Cu") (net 2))
 (segment (start 127.111649 124.499) (end 124.006649 121.394) (width 0.5) (layer "B.Cu") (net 2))
 (segment (start 102.9 124.4017) (end 102.6 124.1017) (width 0.5) (layer "F.Cu") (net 20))
 (segment (start 115.47 122.6) (end 117.5 122.6) (width 0.5) (layer "F.Cu") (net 20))
 (segment (start 113.6683 122.6) (end 111.8666 124.4017) (width 0.5) (layer "F.Cu") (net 20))
 (segment (start 102.6 122.6) (end 102.6 124.1017) (width 0.5) (layer "F.Cu") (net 20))
 (segment (start 132.5002 103.0202) (end 128.3662 103.0202) (width 0.5) (layer "F.Cu") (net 20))
 (segment (start 115.47 122.6) (end 113.6683 122.6) (width 0.5) (layer "F.Cu") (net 20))
 (segment (start 124.2473 107.1391) (end 124.2473 107.7354) (width 0.5) (layer "F.Cu") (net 20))
 (segment (start 128.3662 103.0202) (end 124.2473 107.1391) (width 0.5) (layer "F.Cu") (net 20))
 (segment (start 134.08 104.6) (end 132.5002 103.0202) (width 0.5) (layer "F.Cu") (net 20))
 (segment (start 111.8666 124.4017) (end 102.9 124.4017) (width 0.5) (layer "F.Cu") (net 20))
 (segment (start 117.5 122.6) (end 118.2 121.9) (width 0.5) (layer "F.Cu") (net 20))
 (via (at 124.2473 107.7354) (size 0.9) (drill 0.5) (layers "F.Cu" "B.Cu") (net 20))
 (segment (start 124.2488 109.38) (end 124.7058 109.837) (width 0.5) (layer "B.Cu") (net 20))
 (segment (start 124.7058 116.8229) (end 119.6287 121.9) (width 0.5) (layer "B.Cu") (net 20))
 (segment (start 124.2488 108.3178) (end 124.2488 109.38) (width 0.5) (layer "B.Cu") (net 20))
 (segment (start 124.2473 107.7354) (end 124.2473 108.3163) (width 0.5) (layer "B.Cu") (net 20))
 (segment (start 124.7058 109.837) (end 124.7058 116.8229) (width 0.5) (layer "B.Cu") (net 20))
 (segment (start 124.2473 108.3163) (end 124.2488 108.3178) (width 0.5) (layer "B.Cu") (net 20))
 (segment (start 119.6287 121.9) (end 118.2 121.9) (width 0.5) (layer "B.Cu") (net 20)))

